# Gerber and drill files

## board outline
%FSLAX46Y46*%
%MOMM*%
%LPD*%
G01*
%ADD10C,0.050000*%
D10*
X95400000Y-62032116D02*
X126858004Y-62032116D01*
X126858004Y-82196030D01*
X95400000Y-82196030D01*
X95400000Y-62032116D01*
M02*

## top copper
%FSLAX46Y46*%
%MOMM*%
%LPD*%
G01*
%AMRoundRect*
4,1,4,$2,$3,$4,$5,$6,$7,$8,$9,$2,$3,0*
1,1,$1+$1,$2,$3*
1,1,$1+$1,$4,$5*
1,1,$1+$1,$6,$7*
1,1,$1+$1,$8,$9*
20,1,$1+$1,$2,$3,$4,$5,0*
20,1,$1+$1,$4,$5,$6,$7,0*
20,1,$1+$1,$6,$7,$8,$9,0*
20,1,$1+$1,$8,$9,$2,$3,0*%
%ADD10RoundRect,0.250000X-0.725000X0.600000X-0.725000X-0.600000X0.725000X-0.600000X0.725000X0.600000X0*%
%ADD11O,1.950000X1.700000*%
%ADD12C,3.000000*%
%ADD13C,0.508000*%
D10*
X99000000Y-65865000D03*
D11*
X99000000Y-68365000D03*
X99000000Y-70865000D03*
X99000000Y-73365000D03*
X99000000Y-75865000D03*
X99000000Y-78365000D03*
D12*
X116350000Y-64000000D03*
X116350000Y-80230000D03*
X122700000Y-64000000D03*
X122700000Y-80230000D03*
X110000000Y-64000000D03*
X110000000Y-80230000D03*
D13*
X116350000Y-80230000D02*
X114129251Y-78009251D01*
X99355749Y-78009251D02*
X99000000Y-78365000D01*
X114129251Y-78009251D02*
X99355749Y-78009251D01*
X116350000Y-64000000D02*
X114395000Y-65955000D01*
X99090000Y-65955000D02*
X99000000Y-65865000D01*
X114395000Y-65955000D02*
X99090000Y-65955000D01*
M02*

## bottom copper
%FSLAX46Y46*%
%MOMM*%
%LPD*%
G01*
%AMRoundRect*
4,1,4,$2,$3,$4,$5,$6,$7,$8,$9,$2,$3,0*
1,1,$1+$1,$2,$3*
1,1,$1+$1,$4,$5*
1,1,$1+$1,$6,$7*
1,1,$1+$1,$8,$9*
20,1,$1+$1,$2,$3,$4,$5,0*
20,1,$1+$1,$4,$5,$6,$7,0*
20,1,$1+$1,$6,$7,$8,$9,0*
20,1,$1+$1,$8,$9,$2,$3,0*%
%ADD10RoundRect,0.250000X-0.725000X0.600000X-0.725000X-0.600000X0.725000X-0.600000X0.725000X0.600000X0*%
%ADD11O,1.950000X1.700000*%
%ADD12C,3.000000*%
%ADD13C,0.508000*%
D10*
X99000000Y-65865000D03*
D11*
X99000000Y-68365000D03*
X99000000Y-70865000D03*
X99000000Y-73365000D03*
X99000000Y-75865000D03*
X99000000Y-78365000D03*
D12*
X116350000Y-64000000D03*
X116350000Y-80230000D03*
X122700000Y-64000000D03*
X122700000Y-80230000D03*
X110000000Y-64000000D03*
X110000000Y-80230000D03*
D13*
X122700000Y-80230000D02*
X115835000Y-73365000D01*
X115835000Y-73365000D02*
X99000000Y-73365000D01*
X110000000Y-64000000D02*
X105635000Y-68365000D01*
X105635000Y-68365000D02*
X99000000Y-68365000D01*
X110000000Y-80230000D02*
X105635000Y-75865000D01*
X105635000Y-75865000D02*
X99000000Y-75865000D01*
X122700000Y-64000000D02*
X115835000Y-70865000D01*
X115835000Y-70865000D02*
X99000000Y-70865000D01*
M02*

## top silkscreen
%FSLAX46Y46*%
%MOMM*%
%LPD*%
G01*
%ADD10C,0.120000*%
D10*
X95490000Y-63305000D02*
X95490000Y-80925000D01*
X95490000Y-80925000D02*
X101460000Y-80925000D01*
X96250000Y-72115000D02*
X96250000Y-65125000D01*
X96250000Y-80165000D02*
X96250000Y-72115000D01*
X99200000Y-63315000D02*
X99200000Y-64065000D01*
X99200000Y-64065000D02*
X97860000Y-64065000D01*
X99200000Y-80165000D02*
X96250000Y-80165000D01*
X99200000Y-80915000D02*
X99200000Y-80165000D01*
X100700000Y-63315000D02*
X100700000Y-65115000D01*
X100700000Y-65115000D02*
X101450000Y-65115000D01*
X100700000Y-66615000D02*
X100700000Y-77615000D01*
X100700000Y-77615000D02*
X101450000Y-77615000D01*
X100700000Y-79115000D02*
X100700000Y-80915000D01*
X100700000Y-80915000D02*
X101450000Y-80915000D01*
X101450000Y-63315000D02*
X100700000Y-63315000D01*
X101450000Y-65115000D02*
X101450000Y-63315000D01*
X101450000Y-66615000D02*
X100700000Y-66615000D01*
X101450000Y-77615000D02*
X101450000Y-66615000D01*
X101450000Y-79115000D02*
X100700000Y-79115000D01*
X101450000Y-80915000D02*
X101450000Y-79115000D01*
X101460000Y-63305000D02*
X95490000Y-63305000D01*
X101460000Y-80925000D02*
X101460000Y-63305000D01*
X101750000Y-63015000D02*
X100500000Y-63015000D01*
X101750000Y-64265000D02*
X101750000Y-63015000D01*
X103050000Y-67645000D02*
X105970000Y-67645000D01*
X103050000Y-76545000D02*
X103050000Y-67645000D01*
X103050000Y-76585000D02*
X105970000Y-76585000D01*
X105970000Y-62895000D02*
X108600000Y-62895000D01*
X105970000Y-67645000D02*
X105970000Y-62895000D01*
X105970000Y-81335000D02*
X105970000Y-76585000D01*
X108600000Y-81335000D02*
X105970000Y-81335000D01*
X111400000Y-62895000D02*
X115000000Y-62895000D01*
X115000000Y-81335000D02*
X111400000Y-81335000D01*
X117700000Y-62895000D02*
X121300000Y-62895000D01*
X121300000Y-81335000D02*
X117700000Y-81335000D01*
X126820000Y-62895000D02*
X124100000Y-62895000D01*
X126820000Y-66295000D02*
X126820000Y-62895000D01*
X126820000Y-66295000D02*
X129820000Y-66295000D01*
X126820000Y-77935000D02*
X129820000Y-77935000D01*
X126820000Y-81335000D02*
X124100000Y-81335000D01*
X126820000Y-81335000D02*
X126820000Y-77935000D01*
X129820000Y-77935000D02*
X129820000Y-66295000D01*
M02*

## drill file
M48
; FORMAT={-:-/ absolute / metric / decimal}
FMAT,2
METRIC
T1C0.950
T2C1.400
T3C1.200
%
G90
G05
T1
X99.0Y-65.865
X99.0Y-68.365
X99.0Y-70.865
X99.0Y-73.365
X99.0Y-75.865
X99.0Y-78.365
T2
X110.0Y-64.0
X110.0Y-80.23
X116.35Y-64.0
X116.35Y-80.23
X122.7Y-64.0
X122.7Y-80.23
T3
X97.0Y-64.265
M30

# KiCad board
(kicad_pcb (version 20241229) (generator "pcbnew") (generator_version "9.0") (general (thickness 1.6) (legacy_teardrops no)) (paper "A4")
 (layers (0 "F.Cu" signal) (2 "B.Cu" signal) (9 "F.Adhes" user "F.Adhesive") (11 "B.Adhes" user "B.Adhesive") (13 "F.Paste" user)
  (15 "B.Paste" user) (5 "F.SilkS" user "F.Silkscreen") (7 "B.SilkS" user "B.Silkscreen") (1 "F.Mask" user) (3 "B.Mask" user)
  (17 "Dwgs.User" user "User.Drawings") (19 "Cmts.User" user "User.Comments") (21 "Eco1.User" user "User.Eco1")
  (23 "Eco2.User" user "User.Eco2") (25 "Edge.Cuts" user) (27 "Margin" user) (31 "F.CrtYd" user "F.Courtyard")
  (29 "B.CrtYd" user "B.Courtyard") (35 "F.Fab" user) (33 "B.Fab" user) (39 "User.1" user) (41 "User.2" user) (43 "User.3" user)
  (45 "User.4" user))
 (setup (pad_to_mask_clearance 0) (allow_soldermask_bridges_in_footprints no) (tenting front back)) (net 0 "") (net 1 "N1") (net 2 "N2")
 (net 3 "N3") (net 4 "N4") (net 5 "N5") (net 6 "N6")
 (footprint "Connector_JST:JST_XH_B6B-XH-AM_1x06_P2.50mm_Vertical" (layer "F.Cu") (at 99 65.865 -90)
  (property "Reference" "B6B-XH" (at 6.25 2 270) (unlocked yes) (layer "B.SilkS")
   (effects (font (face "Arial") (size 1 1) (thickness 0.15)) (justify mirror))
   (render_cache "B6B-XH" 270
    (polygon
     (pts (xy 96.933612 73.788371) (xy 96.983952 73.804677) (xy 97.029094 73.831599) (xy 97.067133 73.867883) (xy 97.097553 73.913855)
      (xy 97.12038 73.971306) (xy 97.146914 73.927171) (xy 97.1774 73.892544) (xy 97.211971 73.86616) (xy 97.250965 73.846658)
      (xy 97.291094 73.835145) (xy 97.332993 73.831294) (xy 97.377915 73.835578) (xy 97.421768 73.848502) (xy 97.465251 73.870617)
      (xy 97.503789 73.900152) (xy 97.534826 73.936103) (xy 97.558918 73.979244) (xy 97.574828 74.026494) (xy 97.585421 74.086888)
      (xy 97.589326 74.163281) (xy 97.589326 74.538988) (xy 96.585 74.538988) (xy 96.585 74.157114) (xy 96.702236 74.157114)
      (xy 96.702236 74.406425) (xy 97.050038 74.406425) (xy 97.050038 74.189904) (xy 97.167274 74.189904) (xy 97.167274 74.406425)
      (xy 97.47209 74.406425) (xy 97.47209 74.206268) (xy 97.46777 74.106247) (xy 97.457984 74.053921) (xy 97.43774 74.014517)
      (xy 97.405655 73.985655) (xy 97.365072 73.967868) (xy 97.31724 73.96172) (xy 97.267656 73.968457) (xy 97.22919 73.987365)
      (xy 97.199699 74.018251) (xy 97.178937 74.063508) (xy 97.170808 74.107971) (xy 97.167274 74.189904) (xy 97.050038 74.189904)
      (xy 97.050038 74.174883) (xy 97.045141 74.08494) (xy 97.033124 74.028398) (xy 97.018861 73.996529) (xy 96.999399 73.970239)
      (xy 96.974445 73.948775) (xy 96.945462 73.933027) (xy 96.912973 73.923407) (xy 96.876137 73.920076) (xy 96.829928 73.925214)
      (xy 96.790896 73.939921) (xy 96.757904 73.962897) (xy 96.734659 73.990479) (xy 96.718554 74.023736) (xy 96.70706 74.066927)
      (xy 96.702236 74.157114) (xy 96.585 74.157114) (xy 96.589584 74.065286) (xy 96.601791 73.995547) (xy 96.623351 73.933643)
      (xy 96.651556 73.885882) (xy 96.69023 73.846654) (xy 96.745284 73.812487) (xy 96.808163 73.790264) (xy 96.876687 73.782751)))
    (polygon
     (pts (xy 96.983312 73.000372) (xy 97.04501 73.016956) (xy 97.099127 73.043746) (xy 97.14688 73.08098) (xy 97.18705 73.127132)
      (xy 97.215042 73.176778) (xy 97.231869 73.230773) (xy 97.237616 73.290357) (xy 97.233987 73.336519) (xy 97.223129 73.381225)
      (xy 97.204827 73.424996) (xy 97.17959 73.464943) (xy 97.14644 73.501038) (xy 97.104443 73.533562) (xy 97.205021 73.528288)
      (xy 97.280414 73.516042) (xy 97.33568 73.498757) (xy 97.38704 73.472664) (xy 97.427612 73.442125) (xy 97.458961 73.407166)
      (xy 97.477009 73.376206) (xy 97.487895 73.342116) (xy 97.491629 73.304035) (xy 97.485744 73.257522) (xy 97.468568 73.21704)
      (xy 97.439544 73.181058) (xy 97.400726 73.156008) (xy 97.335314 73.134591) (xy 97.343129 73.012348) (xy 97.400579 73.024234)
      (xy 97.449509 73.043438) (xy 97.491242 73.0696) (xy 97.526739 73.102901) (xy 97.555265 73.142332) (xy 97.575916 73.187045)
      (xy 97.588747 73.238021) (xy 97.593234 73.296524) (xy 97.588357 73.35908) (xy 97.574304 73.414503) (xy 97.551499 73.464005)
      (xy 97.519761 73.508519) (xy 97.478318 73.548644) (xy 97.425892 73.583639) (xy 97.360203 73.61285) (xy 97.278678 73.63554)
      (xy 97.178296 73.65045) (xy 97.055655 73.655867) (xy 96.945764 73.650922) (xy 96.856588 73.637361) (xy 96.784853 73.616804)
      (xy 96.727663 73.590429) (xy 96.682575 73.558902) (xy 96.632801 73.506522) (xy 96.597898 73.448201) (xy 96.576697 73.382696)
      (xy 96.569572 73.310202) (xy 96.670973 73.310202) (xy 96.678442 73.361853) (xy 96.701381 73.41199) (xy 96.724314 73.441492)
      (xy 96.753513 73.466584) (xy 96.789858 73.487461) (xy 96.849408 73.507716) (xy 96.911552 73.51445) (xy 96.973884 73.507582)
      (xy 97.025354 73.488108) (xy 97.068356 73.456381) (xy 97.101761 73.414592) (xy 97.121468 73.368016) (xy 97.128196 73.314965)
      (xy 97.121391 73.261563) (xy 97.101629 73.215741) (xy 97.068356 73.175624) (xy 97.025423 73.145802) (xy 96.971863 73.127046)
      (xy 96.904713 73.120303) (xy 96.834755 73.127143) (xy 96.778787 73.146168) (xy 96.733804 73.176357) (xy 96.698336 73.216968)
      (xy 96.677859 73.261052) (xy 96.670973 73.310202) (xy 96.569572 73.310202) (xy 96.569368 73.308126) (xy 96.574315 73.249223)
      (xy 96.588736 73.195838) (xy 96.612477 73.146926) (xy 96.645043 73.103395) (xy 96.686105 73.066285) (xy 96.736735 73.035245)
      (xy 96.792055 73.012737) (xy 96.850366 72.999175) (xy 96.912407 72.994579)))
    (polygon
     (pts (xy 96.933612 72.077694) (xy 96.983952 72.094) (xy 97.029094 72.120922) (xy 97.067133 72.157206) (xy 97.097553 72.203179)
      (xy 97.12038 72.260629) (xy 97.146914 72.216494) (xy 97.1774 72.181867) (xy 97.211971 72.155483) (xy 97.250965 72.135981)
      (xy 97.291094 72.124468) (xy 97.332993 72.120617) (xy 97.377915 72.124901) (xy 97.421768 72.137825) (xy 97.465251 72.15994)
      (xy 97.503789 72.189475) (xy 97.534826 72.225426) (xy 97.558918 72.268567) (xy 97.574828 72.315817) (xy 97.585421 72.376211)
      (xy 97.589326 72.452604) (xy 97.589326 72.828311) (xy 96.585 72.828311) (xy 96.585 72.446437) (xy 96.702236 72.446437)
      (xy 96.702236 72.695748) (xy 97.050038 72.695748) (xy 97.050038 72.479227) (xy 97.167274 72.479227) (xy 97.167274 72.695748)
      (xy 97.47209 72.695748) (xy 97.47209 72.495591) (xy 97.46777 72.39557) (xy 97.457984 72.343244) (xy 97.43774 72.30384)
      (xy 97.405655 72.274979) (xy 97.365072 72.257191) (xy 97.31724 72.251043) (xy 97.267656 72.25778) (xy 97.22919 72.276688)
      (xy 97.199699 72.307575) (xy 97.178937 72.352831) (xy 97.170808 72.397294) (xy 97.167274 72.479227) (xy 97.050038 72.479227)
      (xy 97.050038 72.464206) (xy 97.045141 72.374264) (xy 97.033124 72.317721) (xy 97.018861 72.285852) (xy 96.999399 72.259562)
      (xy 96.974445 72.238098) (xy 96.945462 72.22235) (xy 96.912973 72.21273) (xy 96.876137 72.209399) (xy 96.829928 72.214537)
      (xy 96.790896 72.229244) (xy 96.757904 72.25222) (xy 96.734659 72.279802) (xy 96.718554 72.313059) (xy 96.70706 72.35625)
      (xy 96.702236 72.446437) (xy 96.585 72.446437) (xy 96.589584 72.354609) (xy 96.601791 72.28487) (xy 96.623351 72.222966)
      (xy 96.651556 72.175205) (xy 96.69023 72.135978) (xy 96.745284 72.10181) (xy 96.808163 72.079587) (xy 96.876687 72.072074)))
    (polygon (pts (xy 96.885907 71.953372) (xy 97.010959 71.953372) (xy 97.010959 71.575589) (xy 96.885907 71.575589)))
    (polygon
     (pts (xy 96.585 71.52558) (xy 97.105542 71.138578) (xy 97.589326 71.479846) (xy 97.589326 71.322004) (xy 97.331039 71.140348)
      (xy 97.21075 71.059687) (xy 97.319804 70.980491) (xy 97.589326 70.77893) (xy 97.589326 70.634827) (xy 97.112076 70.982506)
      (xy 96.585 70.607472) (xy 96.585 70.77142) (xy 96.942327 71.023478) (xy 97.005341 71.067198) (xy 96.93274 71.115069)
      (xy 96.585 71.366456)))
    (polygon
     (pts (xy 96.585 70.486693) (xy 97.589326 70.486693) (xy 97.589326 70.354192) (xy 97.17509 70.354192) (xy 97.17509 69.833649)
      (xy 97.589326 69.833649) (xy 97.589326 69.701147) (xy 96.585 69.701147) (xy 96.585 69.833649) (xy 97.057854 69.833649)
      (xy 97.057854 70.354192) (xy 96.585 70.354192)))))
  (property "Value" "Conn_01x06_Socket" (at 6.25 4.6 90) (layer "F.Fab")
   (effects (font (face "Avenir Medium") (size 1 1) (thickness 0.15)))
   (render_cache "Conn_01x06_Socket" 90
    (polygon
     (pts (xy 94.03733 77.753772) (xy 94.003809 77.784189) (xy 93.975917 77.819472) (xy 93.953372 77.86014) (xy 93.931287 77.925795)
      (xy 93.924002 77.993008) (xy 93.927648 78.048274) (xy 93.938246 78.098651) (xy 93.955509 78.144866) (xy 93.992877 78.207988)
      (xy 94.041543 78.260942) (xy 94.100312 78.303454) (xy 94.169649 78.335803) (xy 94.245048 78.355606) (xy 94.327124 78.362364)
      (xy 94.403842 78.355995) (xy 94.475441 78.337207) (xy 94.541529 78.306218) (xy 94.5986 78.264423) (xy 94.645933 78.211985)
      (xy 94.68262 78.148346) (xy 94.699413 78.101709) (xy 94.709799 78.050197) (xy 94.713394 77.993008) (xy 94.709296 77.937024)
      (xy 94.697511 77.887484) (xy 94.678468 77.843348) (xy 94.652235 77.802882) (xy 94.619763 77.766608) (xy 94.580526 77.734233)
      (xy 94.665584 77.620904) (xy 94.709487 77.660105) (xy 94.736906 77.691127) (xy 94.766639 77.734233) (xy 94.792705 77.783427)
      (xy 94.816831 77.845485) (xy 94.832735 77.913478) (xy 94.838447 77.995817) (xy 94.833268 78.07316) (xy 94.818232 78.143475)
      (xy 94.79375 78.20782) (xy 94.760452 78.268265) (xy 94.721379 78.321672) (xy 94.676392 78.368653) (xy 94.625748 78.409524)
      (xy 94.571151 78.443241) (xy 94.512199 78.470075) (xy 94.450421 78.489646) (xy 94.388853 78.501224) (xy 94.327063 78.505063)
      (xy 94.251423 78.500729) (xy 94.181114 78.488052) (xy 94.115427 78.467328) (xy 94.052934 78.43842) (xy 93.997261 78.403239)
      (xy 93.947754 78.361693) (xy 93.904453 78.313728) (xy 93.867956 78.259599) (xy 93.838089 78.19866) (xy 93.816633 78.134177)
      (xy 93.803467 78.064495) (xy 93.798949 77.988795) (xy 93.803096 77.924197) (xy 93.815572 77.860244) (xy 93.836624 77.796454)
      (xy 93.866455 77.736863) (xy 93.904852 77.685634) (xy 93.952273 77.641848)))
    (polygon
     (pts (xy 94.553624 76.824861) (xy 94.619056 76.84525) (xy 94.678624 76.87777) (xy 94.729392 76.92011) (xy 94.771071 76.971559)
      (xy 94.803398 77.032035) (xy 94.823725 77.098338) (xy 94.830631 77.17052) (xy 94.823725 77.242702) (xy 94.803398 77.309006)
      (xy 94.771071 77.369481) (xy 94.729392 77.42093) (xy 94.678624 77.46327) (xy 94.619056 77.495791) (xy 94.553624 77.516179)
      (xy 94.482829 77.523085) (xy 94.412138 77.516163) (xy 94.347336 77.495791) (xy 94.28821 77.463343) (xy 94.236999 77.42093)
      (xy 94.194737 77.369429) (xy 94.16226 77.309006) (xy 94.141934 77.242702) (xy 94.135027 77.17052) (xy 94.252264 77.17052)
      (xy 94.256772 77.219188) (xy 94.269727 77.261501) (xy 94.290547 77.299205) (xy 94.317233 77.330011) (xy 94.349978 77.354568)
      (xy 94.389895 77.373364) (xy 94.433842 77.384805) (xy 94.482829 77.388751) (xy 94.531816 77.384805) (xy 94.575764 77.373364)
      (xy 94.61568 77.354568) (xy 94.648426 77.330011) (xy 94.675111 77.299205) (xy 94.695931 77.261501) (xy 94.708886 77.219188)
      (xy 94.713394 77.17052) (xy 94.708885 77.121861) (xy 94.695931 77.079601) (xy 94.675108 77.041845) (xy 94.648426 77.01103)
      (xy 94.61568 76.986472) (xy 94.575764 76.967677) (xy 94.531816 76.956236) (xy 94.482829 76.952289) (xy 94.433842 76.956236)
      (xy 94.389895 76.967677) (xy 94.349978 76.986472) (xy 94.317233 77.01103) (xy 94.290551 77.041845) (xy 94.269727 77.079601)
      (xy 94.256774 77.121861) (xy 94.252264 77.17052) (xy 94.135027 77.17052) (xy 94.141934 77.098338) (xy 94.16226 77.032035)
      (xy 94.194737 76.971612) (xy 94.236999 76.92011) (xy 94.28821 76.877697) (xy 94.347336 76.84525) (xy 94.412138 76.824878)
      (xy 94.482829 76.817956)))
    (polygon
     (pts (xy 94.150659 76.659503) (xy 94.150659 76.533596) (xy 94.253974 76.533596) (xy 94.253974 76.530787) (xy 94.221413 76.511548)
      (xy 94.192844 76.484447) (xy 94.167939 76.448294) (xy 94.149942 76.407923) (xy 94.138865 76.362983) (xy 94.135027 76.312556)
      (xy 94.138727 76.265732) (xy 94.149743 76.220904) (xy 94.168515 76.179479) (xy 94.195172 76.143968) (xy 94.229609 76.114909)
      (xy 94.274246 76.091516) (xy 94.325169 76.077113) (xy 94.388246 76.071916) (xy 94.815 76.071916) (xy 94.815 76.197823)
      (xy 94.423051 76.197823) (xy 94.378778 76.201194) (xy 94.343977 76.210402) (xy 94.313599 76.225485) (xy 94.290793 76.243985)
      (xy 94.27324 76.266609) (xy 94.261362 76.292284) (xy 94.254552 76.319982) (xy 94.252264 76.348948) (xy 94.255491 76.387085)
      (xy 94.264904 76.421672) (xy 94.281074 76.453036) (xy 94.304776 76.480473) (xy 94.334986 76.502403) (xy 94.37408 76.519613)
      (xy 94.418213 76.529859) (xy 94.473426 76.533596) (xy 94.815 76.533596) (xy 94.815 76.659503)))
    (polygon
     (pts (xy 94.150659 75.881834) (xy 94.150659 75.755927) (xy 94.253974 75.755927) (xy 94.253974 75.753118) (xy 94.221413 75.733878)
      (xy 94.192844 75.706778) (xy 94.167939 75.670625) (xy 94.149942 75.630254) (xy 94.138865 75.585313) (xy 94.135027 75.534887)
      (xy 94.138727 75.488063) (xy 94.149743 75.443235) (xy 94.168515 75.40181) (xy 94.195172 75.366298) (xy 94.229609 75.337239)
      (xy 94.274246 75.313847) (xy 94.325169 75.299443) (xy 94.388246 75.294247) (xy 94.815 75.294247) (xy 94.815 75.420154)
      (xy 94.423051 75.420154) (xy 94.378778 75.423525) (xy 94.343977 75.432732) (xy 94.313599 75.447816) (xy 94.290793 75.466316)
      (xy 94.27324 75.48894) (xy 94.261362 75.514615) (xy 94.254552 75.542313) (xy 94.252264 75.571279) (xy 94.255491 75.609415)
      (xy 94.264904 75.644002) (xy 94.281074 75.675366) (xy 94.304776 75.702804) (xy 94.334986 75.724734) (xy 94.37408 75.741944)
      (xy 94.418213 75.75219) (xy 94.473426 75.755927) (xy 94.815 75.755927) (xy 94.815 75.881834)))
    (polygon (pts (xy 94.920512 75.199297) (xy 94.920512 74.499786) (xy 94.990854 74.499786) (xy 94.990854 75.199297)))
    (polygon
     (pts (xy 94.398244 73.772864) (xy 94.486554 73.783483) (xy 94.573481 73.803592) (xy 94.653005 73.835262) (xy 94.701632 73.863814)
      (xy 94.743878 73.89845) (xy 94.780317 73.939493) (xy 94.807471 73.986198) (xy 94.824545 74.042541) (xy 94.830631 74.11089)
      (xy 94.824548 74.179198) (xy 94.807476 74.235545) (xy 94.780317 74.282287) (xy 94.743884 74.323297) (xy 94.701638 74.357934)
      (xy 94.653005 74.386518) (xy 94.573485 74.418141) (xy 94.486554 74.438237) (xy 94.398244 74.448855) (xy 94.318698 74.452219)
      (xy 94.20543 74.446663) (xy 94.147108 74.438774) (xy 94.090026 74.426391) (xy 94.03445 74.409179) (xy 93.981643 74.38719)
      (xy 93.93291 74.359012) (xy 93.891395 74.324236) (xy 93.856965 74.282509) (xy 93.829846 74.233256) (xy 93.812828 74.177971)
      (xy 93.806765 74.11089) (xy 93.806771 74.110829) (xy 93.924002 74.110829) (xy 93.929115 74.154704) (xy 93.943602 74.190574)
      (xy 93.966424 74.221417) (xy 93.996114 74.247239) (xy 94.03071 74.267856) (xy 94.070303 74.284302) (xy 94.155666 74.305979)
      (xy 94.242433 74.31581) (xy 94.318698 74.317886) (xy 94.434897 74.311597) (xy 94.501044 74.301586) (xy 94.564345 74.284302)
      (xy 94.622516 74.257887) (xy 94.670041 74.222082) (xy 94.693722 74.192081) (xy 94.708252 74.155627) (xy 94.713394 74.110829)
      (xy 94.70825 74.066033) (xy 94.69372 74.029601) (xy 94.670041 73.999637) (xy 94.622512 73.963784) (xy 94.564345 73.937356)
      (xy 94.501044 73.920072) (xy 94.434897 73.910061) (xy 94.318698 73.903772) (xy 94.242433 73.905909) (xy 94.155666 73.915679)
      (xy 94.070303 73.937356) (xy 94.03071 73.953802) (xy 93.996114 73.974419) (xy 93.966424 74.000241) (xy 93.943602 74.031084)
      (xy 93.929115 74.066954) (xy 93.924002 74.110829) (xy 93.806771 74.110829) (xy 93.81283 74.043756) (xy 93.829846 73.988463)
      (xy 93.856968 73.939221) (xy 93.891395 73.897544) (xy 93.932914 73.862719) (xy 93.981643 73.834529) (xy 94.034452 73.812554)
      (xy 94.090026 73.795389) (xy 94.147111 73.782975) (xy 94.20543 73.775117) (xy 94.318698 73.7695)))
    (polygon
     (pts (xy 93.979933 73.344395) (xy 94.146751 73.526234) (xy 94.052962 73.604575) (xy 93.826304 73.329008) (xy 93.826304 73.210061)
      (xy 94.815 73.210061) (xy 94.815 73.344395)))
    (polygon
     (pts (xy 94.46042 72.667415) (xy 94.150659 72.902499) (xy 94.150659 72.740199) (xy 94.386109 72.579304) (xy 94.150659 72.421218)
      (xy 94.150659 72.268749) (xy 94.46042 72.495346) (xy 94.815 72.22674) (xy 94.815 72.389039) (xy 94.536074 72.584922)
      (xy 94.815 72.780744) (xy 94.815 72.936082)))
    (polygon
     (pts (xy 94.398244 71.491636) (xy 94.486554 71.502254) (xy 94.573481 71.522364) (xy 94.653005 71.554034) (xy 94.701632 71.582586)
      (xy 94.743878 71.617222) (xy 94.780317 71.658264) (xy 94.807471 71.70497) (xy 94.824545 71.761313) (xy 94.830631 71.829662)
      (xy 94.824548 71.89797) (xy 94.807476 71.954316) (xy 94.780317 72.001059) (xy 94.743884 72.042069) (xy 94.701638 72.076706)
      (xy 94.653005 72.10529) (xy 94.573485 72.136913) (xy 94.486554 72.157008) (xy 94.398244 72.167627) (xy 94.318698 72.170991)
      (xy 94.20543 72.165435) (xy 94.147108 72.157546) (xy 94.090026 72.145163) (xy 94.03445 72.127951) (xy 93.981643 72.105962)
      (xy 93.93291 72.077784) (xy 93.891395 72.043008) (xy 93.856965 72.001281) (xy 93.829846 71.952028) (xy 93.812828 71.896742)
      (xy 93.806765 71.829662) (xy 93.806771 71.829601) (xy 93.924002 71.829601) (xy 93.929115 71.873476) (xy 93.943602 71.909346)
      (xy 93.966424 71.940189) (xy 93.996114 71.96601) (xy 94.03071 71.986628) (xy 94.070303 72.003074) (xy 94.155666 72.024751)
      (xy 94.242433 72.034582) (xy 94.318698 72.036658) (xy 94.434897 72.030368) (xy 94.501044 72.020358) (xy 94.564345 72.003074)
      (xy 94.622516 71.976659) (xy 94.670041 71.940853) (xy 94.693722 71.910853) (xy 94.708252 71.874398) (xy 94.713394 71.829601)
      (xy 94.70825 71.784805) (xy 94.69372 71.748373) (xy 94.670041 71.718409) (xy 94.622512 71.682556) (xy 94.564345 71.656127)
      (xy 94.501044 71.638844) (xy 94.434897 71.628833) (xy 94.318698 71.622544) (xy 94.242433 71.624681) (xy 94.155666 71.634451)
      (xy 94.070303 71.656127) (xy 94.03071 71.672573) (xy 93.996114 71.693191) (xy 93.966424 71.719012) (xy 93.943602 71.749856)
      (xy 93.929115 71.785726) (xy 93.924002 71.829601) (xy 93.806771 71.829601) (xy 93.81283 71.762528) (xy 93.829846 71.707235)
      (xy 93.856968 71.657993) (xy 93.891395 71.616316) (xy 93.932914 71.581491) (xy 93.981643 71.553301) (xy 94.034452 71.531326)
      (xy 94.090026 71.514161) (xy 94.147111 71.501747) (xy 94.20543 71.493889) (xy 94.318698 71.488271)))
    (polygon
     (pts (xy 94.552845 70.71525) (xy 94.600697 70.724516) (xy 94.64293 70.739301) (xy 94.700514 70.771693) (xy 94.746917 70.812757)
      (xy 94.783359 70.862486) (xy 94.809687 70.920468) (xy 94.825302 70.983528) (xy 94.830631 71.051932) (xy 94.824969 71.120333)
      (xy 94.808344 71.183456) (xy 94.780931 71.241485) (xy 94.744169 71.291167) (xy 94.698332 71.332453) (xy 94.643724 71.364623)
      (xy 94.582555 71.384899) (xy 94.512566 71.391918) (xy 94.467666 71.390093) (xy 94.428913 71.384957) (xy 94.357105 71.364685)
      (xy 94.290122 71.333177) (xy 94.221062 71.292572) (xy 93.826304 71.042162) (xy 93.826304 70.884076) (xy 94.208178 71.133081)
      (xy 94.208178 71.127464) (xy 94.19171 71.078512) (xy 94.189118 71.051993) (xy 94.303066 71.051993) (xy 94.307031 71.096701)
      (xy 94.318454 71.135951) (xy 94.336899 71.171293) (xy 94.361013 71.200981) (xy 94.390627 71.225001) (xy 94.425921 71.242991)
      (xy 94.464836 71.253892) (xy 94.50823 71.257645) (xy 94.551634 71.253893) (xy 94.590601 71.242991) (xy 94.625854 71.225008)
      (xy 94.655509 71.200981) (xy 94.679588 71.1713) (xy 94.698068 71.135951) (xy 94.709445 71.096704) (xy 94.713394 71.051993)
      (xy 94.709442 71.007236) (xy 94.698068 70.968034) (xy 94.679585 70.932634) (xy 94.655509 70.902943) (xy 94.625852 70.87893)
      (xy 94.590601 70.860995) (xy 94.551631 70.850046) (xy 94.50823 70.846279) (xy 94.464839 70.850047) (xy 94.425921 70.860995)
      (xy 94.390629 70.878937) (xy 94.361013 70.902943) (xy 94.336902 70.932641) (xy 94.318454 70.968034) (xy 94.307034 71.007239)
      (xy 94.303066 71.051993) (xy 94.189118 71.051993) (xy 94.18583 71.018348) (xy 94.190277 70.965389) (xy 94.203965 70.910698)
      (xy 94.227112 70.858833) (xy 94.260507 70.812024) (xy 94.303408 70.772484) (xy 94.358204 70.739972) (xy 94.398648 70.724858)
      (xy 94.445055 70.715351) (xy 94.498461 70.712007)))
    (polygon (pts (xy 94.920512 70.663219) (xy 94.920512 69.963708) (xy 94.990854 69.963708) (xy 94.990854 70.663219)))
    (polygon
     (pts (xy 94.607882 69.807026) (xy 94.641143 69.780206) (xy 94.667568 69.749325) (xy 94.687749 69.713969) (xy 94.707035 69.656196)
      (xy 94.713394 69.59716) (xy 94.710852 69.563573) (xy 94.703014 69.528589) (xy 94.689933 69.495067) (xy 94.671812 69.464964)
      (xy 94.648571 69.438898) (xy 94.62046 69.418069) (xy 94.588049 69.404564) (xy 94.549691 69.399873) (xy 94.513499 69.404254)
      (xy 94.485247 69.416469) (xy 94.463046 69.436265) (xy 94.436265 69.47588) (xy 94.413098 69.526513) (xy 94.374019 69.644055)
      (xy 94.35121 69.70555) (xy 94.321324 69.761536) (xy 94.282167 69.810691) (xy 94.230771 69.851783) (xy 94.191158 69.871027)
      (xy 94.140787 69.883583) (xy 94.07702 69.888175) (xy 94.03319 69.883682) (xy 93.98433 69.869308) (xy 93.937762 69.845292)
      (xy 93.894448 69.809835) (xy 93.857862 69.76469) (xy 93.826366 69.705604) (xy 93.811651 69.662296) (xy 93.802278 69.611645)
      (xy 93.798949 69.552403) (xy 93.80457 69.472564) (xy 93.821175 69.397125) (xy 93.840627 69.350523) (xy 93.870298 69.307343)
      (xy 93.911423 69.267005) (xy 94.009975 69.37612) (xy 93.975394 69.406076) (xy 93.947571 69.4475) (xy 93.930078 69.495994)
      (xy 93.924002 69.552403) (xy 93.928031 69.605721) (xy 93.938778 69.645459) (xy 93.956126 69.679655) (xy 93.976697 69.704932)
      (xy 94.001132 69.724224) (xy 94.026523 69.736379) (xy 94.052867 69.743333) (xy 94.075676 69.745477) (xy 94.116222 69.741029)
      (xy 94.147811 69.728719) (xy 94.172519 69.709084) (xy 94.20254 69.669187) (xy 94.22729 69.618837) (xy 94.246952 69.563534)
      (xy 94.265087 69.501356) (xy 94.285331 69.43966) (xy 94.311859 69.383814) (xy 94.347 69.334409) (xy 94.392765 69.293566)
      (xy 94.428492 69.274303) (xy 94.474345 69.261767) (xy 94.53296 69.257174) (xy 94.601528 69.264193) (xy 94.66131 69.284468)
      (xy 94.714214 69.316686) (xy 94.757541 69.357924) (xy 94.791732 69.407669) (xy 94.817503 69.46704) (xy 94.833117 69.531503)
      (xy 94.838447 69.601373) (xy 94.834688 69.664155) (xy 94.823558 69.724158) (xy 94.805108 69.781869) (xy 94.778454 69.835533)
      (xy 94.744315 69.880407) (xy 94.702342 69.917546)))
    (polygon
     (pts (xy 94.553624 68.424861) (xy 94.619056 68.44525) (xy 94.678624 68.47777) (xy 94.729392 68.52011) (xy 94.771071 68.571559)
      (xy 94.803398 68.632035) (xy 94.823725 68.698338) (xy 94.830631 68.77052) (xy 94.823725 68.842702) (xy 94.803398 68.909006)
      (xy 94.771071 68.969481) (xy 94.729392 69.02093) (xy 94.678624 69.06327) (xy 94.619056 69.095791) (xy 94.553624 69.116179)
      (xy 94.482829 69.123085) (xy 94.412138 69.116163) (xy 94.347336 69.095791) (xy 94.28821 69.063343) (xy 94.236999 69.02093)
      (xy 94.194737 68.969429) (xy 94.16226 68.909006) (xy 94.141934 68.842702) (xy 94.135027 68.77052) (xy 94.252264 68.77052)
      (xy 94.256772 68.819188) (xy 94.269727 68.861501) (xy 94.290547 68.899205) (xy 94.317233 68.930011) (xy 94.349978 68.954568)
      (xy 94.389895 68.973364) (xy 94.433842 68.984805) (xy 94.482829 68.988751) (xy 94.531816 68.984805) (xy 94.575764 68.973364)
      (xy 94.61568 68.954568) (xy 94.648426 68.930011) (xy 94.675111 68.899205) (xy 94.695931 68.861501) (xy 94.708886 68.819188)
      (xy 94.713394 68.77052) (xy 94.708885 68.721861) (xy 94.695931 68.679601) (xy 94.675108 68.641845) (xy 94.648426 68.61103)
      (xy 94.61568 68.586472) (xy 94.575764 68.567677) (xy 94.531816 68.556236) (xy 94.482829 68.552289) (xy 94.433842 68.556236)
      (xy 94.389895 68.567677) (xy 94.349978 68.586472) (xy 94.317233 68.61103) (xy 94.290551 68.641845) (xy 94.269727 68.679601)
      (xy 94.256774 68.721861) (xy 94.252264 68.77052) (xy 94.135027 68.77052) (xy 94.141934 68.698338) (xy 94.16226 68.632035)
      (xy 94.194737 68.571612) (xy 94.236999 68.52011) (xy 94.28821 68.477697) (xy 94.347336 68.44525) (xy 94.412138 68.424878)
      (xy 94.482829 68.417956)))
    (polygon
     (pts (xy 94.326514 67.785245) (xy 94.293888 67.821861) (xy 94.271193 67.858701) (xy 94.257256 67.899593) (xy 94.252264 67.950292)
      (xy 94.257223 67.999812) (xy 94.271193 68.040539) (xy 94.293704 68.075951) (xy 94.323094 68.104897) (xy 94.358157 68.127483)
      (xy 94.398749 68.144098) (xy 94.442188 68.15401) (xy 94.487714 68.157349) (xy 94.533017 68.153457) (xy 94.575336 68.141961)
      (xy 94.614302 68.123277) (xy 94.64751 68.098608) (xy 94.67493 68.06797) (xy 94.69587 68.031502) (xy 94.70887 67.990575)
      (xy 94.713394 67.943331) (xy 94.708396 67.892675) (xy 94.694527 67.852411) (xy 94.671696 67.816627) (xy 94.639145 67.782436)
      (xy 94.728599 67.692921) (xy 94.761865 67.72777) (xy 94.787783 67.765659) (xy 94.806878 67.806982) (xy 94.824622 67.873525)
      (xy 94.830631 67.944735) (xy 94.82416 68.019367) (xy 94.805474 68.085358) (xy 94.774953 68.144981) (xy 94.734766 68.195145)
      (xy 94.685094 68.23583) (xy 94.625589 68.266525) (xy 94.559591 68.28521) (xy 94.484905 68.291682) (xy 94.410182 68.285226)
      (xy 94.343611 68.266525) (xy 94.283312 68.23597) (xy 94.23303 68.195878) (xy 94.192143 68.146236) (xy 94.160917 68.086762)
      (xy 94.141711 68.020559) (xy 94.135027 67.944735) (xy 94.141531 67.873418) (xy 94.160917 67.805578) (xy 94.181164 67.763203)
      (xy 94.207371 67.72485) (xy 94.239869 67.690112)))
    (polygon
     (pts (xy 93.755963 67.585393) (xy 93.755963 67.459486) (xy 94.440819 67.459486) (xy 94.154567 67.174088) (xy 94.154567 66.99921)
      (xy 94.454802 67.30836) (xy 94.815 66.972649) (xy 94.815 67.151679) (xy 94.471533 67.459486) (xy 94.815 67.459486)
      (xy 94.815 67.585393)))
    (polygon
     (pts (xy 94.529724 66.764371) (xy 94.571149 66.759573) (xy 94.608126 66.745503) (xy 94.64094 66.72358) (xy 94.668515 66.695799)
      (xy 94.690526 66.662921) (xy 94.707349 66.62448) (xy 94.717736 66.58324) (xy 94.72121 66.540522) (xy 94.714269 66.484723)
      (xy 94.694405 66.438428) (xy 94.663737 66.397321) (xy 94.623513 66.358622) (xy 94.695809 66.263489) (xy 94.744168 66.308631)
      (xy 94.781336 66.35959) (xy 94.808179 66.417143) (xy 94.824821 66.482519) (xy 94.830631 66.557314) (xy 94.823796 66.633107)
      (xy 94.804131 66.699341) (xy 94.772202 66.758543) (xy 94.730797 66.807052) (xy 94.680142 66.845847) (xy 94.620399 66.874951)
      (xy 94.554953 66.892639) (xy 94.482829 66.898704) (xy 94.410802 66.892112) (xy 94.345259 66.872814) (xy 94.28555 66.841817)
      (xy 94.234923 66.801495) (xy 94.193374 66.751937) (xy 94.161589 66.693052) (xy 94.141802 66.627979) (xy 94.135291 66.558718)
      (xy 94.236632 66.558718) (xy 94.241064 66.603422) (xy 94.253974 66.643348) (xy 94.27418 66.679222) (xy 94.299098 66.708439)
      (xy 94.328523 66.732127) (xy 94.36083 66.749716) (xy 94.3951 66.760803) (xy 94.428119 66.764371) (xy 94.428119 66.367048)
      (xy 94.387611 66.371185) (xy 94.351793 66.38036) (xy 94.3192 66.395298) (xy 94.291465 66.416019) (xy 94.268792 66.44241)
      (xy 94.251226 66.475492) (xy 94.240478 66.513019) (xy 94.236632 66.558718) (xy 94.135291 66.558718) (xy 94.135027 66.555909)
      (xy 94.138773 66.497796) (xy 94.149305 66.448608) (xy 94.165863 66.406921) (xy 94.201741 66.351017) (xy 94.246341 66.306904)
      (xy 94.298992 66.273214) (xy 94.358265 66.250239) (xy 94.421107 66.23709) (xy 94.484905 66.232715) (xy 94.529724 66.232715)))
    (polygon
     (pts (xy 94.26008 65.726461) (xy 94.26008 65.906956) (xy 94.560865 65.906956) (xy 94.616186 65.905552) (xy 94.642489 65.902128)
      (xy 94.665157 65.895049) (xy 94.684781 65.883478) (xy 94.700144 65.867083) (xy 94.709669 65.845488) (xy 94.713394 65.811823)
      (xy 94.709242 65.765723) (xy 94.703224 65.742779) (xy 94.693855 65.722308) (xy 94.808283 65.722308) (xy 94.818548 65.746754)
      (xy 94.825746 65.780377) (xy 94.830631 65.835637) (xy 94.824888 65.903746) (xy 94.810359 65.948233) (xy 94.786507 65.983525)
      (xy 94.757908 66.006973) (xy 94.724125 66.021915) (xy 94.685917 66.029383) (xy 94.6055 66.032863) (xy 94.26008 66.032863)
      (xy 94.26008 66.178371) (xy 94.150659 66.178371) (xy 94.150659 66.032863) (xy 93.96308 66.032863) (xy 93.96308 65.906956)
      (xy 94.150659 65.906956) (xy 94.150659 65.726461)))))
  (fp_line (start -2.56 3.51) (end 15.06 3.51) (stroke (width 0.12) (type solid)) (layer "F.SilkS"))
  (fp_line (start 15.06 3.51) (end 15.06 -2.46) (stroke (width 0.12) (type solid)) (layer "F.SilkS"))
  (fp_line (start 6.25 2.75) (end -0.74 2.75) (stroke (width 0.12) (type solid)) (layer "F.SilkS"))
  (fp_line (start 14.3 2.75) (end 6.25 2.75) (stroke (width 0.12) (type solid)) (layer "F.SilkS"))
  (fp_line (start -2.55 -0.2) (end -1.8 -0.2) (stroke (width 0.12) (type solid)) (layer "F.SilkS"))
  (fp_line (start -1.8 -0.2) (end -1.8 1.14) (stroke (width 0.12) (type solid)) (layer "F.SilkS"))
  (fp_line (start 14.3 -0.2) (end 14.3 2.75) (stroke (width 0.12) (type solid)) (layer "F.SilkS"))
  (fp_line (start 15.05 -0.2) (end 14.3 -0.2) (stroke (width 0.12) (type solid)) (layer "F.SilkS"))
  (fp_line (start -2.55 -1.7) (end -0.75 -1.7) (stroke (width 0.12) (type solid)) (layer "F.SilkS"))
  (fp_line (start -0.75 -1.7) (end -0.75 -2.45) (stroke (width 0.12) (type solid)) (layer "F.SilkS"))
  (fp_line (start 0.75 -1.7) (end 11.75 -1.7) (stroke (width 0.12) (type solid)) (layer "F.SilkS"))
  (fp_line (start 11.75 -1.7) (end 11.75 -2.45) (stroke (width 0.12) (type solid)) (layer "F.SilkS"))
  (fp_line (start 13.25 -1.7) (end 15.05 -1.7) (stroke (width 0.12) (type solid)) (layer "F.SilkS"))
  (fp_line (start 15.05 -1.7) (end 15.05 -2.45) (stroke (width 0.12) (type solid)) (layer "F.SilkS"))
  (fp_line (start -2.55 -2.45) (end -2.55 -1.7) (stroke (width 0.12) (type solid)) (layer "F.SilkS"))
  (fp_line (start -0.75 -2.45) (end -2.55 -2.45) (stroke (width 0.12) (type solid)) (layer "F.SilkS"))
  (fp_line (start 0.75 -2.45) (end 0.75 -1.7) (stroke (width 0.12) (type solid)) (layer "F.SilkS"))
  (fp_line (start 11.75 -2.45) (end 0.75 -2.45) (stroke (width 0.12) (type solid)) (layer "F.SilkS"))
  (fp_line (start 13.25 -2.45) (end 13.25 -1.7) (stroke (width 0.12) (type solid)) (layer "F.SilkS"))
  (fp_line (start 15.05 -2.45) (end 13.25 -2.45) (stroke (width 0.12) (type solid)) (layer "F.SilkS"))
  (fp_line (start -2.56 -2.46) (end -2.56 3.51) (stroke (width 0.12) (type solid)) (layer "F.SilkS"))
  (fp_line (start 15.06 -2.46) (end -2.56 -2.46) (stroke (width 0.12) (type solid)) (layer "F.SilkS"))
  (fp_line (start -2.85 -2.75) (end -2.85 -1.5) (stroke (width 0.12) (type solid)) (layer "F.SilkS"))
  (fp_line (start -1.6 -2.75) (end -2.85 -2.75) (stroke (width 0.12) (type solid)) (layer "F.SilkS"))
  (pad "" np_thru_hole circle (at -1.6 2 270) (size 1.2 1.2) (drill 1.2) (layers "*.Cu" "*.Mask"))
  (pad "1" thru_hole roundrect (at 0 0 270) (size 1.7 1.95) (drill 0.95) (layers "*.Cu" "*.Mask") (remove_unused_layers no)
   (roundrect_rratio 0.147059) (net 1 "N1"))
  (pad "2" thru_hole oval (at 2.5 0 270) (size 1.7 1.95) (drill 0.95) (layers "*.Cu" "*.Mask") (remove_unused_layers no) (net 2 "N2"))
  (pad "3" thru_hole oval (at 5 0 270) (size 1.7 1.95) (drill 0.95) (layers "*.Cu" "*.Mask") (remove_unused_layers no) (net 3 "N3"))
  (pad "4" thru_hole oval (at 7.5 0 270) (size 1.7 1.95) (drill 0.95) (layers "*.Cu" "*.Mask") (remove_unused_layers no) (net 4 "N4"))
  (pad "5" thru_hole oval (at 10 0 270) (size 1.7 1.95) (drill 0.95) (layers "*.Cu" "*.Mask") (remove_unused_layers no) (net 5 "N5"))
  (pad "6" thru_hole oval (at 12.5 0 270) (size 1.7 1.95) (drill 0.95) (layers "*.Cu" "*.Mask") (remove_unused_layers no) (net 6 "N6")))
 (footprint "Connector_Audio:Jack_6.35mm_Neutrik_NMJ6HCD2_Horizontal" (layer "F.Cu") (at 110 64)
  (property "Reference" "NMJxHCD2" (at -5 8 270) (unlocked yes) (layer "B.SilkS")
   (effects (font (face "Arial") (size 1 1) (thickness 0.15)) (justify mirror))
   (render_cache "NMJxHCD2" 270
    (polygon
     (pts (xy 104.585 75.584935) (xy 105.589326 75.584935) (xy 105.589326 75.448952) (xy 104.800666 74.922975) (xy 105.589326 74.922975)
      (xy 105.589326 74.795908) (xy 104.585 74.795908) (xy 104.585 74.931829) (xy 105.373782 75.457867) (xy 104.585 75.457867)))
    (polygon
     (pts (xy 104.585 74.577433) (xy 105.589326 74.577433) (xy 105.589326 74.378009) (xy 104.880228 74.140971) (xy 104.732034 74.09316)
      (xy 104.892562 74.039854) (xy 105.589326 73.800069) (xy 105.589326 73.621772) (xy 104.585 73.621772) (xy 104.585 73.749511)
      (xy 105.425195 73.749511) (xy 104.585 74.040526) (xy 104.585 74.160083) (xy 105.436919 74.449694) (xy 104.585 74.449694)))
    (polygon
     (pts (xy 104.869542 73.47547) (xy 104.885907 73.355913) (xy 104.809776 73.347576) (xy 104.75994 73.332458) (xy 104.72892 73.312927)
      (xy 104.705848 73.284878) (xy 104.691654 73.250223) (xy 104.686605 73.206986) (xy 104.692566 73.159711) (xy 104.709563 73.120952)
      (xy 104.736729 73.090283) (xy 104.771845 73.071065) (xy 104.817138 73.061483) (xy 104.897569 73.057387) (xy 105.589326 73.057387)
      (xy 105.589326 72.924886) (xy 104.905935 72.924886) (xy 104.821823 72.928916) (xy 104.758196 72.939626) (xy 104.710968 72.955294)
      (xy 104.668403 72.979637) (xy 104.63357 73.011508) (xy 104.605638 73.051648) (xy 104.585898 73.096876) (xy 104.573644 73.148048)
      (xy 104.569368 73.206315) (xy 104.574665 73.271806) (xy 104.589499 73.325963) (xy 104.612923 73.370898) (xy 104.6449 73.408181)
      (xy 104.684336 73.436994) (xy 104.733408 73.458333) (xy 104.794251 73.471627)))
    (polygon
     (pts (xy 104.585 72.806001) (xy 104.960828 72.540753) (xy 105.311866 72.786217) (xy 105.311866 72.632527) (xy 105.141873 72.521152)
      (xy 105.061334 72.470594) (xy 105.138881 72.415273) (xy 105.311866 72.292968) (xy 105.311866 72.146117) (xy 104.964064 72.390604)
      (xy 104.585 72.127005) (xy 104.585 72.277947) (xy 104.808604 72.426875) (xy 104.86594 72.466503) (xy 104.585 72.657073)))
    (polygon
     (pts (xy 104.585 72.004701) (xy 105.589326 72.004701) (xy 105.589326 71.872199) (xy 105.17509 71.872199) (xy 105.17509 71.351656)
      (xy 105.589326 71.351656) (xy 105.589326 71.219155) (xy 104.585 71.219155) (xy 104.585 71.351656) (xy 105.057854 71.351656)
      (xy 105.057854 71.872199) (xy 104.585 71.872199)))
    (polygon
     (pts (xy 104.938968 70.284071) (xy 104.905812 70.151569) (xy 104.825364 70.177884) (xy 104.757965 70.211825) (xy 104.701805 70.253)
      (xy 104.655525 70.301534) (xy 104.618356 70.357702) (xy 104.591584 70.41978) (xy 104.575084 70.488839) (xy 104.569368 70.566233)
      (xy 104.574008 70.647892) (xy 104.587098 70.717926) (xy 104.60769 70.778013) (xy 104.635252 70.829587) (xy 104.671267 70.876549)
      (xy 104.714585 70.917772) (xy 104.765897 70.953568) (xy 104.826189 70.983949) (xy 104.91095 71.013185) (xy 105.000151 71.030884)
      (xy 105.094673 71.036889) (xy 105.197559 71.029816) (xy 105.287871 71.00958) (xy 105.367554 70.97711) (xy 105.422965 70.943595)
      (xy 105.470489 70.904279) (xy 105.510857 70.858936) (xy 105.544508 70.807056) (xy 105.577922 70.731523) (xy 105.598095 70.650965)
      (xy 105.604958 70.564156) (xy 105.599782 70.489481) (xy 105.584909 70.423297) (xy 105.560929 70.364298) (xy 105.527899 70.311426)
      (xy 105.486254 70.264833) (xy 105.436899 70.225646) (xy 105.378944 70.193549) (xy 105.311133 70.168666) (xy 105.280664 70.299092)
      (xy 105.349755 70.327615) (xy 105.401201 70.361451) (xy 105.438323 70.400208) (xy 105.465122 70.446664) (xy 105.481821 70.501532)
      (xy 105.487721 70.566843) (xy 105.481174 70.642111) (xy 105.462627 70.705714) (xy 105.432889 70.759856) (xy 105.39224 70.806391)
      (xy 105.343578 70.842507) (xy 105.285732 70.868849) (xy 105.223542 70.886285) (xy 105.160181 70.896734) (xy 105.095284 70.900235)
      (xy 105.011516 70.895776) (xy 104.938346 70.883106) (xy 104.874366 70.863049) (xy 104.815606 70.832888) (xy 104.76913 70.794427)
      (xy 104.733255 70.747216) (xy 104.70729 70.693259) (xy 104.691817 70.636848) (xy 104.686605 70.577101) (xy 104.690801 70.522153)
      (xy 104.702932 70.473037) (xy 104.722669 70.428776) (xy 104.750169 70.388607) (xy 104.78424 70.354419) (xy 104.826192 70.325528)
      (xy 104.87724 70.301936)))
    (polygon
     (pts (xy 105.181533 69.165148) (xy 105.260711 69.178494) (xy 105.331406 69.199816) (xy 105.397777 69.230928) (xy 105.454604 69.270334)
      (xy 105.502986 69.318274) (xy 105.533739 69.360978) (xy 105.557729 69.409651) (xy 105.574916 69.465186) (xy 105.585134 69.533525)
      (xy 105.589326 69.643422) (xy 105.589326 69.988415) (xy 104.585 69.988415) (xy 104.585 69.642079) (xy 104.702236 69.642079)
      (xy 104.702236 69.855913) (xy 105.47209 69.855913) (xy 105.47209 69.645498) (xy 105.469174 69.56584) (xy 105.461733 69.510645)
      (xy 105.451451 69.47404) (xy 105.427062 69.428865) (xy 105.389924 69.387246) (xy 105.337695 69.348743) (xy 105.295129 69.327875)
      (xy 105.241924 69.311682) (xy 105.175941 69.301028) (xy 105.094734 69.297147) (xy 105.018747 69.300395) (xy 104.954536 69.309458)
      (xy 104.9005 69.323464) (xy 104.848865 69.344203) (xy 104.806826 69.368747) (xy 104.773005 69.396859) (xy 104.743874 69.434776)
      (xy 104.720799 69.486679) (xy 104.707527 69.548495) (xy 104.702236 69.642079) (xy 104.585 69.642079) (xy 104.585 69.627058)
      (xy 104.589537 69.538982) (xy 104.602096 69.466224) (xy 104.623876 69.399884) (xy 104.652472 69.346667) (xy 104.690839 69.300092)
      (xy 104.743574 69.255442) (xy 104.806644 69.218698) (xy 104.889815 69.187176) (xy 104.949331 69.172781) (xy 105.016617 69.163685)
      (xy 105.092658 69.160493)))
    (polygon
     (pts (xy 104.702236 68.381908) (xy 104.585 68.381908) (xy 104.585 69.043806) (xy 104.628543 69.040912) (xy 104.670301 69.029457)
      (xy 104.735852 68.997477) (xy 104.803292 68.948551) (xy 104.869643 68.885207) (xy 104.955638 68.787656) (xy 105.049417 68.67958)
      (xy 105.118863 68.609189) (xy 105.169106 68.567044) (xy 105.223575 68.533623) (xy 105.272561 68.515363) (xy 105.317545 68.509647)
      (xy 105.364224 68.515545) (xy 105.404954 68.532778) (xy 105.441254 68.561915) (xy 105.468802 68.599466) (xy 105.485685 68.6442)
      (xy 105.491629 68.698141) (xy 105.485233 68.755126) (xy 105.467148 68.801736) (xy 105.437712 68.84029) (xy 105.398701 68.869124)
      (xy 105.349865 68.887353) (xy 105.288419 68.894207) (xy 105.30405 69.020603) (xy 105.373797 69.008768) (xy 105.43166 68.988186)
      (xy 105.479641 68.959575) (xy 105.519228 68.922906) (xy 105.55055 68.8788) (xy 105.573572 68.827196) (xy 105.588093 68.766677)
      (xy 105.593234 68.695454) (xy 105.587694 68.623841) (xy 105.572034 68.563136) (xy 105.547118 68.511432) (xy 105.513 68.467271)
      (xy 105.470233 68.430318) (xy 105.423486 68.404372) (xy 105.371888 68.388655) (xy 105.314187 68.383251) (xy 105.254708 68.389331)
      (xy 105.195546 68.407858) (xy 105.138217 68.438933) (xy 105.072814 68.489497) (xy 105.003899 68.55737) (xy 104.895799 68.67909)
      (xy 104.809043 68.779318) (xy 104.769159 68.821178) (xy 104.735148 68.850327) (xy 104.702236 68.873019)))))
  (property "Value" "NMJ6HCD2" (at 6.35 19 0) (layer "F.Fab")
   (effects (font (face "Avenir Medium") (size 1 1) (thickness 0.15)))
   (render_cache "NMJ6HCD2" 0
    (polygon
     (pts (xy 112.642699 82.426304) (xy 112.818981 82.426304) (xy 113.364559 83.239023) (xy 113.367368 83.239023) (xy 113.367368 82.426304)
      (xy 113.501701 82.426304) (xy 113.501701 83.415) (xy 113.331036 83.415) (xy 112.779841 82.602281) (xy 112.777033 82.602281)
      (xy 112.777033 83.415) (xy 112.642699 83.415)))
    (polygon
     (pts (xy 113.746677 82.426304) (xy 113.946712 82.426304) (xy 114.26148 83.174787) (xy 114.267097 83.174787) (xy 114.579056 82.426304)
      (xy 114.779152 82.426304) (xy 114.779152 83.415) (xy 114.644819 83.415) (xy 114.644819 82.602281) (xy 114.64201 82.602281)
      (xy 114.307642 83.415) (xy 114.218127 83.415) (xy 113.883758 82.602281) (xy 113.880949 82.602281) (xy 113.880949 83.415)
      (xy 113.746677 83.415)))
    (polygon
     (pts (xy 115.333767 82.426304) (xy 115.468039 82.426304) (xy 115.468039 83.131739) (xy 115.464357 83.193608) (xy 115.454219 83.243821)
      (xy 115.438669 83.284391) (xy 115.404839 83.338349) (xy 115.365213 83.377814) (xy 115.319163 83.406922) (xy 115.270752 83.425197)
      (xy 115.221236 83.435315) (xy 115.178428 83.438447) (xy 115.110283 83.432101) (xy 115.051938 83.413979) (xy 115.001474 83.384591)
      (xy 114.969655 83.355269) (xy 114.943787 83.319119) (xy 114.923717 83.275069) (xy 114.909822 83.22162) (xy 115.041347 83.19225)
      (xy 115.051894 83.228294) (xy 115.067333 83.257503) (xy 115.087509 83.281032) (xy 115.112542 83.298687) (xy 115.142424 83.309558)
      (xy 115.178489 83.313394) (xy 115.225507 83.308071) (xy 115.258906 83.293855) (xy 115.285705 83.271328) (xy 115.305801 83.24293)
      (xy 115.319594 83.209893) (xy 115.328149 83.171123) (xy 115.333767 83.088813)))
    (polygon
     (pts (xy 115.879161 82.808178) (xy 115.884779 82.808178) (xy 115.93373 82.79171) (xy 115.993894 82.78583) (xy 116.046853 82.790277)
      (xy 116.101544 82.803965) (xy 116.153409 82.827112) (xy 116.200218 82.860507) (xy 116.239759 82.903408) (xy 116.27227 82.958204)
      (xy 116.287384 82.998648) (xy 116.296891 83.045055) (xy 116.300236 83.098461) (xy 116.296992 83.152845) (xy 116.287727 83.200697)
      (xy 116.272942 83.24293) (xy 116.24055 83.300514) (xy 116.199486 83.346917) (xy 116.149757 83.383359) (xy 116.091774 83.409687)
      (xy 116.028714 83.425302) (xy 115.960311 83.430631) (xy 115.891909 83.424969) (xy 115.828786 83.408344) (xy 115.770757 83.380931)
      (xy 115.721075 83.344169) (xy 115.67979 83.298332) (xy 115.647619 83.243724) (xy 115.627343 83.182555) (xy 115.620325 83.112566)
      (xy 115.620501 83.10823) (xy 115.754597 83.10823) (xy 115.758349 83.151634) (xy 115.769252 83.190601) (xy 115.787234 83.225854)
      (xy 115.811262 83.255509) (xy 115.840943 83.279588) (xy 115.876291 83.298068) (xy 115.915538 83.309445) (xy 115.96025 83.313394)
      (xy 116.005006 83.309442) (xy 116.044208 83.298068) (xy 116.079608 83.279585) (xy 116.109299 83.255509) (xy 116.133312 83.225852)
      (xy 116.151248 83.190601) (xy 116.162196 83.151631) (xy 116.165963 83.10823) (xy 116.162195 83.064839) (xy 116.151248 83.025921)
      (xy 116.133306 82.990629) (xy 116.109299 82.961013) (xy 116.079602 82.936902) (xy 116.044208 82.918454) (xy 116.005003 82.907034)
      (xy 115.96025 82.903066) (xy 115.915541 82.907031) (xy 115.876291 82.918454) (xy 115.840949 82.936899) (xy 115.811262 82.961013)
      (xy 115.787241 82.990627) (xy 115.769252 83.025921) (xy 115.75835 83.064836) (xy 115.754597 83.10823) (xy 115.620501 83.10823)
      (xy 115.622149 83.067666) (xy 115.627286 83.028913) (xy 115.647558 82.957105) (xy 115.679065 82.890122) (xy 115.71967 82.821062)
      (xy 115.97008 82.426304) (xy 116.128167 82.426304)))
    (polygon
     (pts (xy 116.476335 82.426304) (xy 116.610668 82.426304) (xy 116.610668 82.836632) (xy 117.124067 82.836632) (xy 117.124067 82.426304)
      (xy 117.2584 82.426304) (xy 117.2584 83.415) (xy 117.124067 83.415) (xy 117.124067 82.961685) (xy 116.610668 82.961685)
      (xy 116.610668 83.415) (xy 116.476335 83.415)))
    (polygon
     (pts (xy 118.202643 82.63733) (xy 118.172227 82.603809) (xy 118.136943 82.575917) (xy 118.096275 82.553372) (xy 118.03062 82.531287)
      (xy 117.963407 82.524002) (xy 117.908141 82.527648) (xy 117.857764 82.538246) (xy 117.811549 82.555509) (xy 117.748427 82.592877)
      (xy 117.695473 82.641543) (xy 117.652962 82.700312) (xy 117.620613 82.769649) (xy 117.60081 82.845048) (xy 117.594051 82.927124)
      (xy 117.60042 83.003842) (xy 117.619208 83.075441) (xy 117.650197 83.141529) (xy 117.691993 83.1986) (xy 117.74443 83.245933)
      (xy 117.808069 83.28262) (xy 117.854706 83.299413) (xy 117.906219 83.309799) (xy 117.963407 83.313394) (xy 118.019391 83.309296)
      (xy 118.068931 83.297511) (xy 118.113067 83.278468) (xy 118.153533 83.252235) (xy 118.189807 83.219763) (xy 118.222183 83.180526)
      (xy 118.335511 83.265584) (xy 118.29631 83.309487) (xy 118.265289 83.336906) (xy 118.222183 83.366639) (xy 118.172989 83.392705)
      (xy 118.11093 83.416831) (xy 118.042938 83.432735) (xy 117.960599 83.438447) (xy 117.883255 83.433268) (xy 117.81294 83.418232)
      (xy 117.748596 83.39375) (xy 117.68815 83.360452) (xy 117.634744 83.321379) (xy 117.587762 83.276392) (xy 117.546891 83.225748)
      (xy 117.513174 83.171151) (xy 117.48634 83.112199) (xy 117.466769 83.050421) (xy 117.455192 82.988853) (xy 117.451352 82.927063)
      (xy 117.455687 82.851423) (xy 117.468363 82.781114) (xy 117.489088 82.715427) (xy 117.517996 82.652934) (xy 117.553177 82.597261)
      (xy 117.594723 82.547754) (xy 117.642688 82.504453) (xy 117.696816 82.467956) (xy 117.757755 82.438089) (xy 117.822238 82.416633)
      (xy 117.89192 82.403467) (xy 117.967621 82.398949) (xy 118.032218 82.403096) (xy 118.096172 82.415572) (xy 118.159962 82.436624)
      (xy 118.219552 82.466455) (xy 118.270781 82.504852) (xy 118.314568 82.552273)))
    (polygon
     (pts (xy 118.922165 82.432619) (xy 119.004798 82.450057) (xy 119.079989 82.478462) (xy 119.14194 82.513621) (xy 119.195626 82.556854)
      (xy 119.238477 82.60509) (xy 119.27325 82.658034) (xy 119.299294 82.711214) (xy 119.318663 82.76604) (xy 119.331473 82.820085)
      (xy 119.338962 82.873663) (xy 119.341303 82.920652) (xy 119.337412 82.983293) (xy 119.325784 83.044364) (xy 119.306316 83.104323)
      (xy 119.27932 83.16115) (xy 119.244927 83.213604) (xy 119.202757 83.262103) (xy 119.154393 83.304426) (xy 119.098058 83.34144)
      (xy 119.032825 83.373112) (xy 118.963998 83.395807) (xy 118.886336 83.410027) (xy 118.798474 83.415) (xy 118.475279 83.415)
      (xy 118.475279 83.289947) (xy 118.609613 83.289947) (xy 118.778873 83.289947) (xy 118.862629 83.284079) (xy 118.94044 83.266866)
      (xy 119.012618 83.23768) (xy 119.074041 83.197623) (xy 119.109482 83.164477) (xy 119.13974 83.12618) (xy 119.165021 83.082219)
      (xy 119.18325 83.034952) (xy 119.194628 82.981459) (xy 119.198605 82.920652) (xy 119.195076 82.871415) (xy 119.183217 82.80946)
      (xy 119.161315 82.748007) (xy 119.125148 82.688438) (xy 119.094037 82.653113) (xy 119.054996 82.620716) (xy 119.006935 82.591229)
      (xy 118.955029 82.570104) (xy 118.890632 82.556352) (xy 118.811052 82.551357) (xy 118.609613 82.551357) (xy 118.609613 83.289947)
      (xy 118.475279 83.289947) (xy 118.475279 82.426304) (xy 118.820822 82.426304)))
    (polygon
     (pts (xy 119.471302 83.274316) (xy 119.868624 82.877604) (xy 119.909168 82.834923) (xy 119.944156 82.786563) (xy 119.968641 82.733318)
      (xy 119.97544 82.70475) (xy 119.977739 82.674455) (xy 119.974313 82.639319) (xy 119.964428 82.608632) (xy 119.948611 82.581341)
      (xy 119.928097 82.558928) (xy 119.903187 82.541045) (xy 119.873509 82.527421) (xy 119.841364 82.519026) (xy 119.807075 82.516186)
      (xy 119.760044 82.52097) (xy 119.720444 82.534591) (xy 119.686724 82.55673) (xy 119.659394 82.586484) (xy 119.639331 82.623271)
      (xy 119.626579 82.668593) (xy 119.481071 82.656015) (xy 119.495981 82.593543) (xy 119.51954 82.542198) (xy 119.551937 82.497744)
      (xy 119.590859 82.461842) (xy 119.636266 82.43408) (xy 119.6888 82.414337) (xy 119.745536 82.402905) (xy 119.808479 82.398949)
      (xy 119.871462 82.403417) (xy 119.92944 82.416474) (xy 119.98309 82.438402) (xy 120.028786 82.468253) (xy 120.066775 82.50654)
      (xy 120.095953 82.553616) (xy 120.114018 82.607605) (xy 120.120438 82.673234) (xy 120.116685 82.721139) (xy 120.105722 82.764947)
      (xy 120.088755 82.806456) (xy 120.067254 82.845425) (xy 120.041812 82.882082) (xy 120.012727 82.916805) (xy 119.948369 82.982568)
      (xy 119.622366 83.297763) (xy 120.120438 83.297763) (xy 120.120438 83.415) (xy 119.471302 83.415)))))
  (fp_line (start -6.95 3.645) (end -4.03 3.645) (stroke (width 0.12) (type solid)) (layer "F.SilkS"))
  (fp_line (start -6.95 12.545) (end -6.95 3.645) (stroke (width 0.12) (type solid)) (layer "F.SilkS"))
  (fp_line (start -6.95 12.585) (end -4.03 12.585) (stroke (width 0.12) (type solid)) (layer "F.SilkS"))
  (fp_line (start -4.03 -1.105) (end -1.4 -1.105) (stroke (width 0.12) (type solid)) (layer "F.SilkS"))
  (fp_line (start -4.03 3.645) (end -4.03 -1.105) (stroke (width 0.12) (type solid)) (layer "F.SilkS"))
  (fp_line (start -4.03 17.335) (end -4.03 12.585) (stroke (width 0.12) (type solid)) (layer "F.SilkS"))
  (fp_line (start -1.4 17.335) (end -4.03 17.335) (stroke (width 0.12) (type solid)) (layer "F.SilkS"))
  (fp_line (start 1.4 -1.105) (end 5 -1.105) (stroke (width 0.12) (type solid)) (layer "F.SilkS"))
  (fp_line (start 5 17.335) (end 1.4 17.335) (stroke (width 0.12) (type solid)) (layer "F.SilkS"))
  (fp_line (start 7.7 -1.105) (end 11.3 -1.105) (stroke (width 0.12) (type solid)) (layer "F.SilkS"))
  (fp_line (start 11.3 17.335) (end 7.7 17.335) (stroke (width 0.12) (type solid)) (layer "F.SilkS"))
  (fp_line (start 16.82 -1.105) (end 14.1 -1.105) (stroke (width 0.12) (type solid)) (layer "F.SilkS"))
  (fp_line (start 16.82 2.295) (end 16.82 -1.105) (stroke (width 0.12) (type solid)) (layer "F.SilkS"))
  (fp_line (start 16.82 2.295) (end 19.82 2.295) (stroke (width 0.12) (type solid)) (layer "F.SilkS"))
  (fp_line (start 16.82 13.935) (end 19.82 13.935) (stroke (width 0.12) (type solid)) (layer "F.SilkS"))
  (fp_line (start 16.82 17.335) (end 14.1 17.335) (stroke (width 0.12) (type solid)) (layer "F.SilkS"))
  (fp_line (start 16.82 17.335) (end 16.82 13.935) (stroke (width 0.12) (type solid)) (layer "F.SilkS"))
  (fp_line (start 19.82 13.935) (end 19.82 2.295) (stroke (width 0.12) (type solid)) (layer "F.SilkS"))
  (pad "R" thru_hole circle (at 6.35 0) (size 3 3) (drill 1.4) (layers "*.Cu" "*.Mask") (remove_unused_layers no) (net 1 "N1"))
  (pad "RN" thru_hole circle (at 6.35 16.23) (size 3 3) (drill 1.4) (layers "*.Cu" "*.Mask") (remove_unused_layers no) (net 6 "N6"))
  (pad "S" thru_hole circle (at 12.7 0) (size 3 3) (drill 1.4) (layers "*.Cu" "*.Mask") (remove_unused_layers no) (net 3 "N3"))
  (pad "SN" thru_hole circle (at 12.7 16.23) (size 3 3) (drill 1.4) (layers "*.Cu" "*.Mask") (remove_unused_layers no) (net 4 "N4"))
  (pad "T" thru_hole circle (at 0 0) (size 3 3) (drill 1.4) (layers "*.Cu" "*.Mask") (remove_unused_layers no) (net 2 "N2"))
  (pad "TN" thru_hole circle (at 0 16.23) (size 3 3) (drill 1.4) (layers "*.Cu" "*.Mask") (remove_unused_layers no) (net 5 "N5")))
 (gr_rect (start 95.4 62.032116) (end 126.858004 82.19603) (stroke (width 0.05) (type solid)) (fill no) (layer "Edge.Cuts"))
 (segment (start 122.7 80.23) (end 115.835 73.365) (width 0.508) (layer "B.Cu") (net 4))
 (segment (start 115.835 73.365) (end 99 73.365) (width 0.508) (layer "B.Cu") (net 4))
 (segment (start 116.35 80.23) (end 114.129251 78.009251) (width 0.508) (layer "F.Cu") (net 6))
 (segment (start 99.355749 78.009251) (end 99 78.365) (width 0.508) (layer "F.Cu") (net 6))
 (segment (start 114.129251 78.009251) (end 99.355749 78.009251) (width 0.508) (layer "F.Cu") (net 6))
 (segment (start 110 64) (end 105.635 68.365) (width 0.508) (layer "B.Cu") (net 2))
 (segment (start 105.635 68.365) (end 99 68.365) (width 0.508) (layer "B.Cu") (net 2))
 (segment (start 116.35 64) (end 114.395 65.955) (width 0.508) (layer "F.Cu") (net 1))
 (segment (start 99.09 65.955) (end 99 65.865) (width 0.508) (layer "F.Cu") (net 1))
 (segment (start 114.395 65.955) (end 99.09 65.955) (width 0.508) (layer "F.Cu") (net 1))
 (segment (start 110 80.23) (end 105.635 75.865) (width 0.508) (layer "B.Cu") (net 5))
 (segment (start 105.635 75.865) (end 99 75.865) (width 0.508) (layer "B.Cu") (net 5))
 (segment (start 122.7 64) (end 115.835 70.865) (width 0.508) (layer "B.Cu") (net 3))
 (segment (start 115.835 70.865) (end 99 70.865) (width 0.508) (layer "B.Cu") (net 3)))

